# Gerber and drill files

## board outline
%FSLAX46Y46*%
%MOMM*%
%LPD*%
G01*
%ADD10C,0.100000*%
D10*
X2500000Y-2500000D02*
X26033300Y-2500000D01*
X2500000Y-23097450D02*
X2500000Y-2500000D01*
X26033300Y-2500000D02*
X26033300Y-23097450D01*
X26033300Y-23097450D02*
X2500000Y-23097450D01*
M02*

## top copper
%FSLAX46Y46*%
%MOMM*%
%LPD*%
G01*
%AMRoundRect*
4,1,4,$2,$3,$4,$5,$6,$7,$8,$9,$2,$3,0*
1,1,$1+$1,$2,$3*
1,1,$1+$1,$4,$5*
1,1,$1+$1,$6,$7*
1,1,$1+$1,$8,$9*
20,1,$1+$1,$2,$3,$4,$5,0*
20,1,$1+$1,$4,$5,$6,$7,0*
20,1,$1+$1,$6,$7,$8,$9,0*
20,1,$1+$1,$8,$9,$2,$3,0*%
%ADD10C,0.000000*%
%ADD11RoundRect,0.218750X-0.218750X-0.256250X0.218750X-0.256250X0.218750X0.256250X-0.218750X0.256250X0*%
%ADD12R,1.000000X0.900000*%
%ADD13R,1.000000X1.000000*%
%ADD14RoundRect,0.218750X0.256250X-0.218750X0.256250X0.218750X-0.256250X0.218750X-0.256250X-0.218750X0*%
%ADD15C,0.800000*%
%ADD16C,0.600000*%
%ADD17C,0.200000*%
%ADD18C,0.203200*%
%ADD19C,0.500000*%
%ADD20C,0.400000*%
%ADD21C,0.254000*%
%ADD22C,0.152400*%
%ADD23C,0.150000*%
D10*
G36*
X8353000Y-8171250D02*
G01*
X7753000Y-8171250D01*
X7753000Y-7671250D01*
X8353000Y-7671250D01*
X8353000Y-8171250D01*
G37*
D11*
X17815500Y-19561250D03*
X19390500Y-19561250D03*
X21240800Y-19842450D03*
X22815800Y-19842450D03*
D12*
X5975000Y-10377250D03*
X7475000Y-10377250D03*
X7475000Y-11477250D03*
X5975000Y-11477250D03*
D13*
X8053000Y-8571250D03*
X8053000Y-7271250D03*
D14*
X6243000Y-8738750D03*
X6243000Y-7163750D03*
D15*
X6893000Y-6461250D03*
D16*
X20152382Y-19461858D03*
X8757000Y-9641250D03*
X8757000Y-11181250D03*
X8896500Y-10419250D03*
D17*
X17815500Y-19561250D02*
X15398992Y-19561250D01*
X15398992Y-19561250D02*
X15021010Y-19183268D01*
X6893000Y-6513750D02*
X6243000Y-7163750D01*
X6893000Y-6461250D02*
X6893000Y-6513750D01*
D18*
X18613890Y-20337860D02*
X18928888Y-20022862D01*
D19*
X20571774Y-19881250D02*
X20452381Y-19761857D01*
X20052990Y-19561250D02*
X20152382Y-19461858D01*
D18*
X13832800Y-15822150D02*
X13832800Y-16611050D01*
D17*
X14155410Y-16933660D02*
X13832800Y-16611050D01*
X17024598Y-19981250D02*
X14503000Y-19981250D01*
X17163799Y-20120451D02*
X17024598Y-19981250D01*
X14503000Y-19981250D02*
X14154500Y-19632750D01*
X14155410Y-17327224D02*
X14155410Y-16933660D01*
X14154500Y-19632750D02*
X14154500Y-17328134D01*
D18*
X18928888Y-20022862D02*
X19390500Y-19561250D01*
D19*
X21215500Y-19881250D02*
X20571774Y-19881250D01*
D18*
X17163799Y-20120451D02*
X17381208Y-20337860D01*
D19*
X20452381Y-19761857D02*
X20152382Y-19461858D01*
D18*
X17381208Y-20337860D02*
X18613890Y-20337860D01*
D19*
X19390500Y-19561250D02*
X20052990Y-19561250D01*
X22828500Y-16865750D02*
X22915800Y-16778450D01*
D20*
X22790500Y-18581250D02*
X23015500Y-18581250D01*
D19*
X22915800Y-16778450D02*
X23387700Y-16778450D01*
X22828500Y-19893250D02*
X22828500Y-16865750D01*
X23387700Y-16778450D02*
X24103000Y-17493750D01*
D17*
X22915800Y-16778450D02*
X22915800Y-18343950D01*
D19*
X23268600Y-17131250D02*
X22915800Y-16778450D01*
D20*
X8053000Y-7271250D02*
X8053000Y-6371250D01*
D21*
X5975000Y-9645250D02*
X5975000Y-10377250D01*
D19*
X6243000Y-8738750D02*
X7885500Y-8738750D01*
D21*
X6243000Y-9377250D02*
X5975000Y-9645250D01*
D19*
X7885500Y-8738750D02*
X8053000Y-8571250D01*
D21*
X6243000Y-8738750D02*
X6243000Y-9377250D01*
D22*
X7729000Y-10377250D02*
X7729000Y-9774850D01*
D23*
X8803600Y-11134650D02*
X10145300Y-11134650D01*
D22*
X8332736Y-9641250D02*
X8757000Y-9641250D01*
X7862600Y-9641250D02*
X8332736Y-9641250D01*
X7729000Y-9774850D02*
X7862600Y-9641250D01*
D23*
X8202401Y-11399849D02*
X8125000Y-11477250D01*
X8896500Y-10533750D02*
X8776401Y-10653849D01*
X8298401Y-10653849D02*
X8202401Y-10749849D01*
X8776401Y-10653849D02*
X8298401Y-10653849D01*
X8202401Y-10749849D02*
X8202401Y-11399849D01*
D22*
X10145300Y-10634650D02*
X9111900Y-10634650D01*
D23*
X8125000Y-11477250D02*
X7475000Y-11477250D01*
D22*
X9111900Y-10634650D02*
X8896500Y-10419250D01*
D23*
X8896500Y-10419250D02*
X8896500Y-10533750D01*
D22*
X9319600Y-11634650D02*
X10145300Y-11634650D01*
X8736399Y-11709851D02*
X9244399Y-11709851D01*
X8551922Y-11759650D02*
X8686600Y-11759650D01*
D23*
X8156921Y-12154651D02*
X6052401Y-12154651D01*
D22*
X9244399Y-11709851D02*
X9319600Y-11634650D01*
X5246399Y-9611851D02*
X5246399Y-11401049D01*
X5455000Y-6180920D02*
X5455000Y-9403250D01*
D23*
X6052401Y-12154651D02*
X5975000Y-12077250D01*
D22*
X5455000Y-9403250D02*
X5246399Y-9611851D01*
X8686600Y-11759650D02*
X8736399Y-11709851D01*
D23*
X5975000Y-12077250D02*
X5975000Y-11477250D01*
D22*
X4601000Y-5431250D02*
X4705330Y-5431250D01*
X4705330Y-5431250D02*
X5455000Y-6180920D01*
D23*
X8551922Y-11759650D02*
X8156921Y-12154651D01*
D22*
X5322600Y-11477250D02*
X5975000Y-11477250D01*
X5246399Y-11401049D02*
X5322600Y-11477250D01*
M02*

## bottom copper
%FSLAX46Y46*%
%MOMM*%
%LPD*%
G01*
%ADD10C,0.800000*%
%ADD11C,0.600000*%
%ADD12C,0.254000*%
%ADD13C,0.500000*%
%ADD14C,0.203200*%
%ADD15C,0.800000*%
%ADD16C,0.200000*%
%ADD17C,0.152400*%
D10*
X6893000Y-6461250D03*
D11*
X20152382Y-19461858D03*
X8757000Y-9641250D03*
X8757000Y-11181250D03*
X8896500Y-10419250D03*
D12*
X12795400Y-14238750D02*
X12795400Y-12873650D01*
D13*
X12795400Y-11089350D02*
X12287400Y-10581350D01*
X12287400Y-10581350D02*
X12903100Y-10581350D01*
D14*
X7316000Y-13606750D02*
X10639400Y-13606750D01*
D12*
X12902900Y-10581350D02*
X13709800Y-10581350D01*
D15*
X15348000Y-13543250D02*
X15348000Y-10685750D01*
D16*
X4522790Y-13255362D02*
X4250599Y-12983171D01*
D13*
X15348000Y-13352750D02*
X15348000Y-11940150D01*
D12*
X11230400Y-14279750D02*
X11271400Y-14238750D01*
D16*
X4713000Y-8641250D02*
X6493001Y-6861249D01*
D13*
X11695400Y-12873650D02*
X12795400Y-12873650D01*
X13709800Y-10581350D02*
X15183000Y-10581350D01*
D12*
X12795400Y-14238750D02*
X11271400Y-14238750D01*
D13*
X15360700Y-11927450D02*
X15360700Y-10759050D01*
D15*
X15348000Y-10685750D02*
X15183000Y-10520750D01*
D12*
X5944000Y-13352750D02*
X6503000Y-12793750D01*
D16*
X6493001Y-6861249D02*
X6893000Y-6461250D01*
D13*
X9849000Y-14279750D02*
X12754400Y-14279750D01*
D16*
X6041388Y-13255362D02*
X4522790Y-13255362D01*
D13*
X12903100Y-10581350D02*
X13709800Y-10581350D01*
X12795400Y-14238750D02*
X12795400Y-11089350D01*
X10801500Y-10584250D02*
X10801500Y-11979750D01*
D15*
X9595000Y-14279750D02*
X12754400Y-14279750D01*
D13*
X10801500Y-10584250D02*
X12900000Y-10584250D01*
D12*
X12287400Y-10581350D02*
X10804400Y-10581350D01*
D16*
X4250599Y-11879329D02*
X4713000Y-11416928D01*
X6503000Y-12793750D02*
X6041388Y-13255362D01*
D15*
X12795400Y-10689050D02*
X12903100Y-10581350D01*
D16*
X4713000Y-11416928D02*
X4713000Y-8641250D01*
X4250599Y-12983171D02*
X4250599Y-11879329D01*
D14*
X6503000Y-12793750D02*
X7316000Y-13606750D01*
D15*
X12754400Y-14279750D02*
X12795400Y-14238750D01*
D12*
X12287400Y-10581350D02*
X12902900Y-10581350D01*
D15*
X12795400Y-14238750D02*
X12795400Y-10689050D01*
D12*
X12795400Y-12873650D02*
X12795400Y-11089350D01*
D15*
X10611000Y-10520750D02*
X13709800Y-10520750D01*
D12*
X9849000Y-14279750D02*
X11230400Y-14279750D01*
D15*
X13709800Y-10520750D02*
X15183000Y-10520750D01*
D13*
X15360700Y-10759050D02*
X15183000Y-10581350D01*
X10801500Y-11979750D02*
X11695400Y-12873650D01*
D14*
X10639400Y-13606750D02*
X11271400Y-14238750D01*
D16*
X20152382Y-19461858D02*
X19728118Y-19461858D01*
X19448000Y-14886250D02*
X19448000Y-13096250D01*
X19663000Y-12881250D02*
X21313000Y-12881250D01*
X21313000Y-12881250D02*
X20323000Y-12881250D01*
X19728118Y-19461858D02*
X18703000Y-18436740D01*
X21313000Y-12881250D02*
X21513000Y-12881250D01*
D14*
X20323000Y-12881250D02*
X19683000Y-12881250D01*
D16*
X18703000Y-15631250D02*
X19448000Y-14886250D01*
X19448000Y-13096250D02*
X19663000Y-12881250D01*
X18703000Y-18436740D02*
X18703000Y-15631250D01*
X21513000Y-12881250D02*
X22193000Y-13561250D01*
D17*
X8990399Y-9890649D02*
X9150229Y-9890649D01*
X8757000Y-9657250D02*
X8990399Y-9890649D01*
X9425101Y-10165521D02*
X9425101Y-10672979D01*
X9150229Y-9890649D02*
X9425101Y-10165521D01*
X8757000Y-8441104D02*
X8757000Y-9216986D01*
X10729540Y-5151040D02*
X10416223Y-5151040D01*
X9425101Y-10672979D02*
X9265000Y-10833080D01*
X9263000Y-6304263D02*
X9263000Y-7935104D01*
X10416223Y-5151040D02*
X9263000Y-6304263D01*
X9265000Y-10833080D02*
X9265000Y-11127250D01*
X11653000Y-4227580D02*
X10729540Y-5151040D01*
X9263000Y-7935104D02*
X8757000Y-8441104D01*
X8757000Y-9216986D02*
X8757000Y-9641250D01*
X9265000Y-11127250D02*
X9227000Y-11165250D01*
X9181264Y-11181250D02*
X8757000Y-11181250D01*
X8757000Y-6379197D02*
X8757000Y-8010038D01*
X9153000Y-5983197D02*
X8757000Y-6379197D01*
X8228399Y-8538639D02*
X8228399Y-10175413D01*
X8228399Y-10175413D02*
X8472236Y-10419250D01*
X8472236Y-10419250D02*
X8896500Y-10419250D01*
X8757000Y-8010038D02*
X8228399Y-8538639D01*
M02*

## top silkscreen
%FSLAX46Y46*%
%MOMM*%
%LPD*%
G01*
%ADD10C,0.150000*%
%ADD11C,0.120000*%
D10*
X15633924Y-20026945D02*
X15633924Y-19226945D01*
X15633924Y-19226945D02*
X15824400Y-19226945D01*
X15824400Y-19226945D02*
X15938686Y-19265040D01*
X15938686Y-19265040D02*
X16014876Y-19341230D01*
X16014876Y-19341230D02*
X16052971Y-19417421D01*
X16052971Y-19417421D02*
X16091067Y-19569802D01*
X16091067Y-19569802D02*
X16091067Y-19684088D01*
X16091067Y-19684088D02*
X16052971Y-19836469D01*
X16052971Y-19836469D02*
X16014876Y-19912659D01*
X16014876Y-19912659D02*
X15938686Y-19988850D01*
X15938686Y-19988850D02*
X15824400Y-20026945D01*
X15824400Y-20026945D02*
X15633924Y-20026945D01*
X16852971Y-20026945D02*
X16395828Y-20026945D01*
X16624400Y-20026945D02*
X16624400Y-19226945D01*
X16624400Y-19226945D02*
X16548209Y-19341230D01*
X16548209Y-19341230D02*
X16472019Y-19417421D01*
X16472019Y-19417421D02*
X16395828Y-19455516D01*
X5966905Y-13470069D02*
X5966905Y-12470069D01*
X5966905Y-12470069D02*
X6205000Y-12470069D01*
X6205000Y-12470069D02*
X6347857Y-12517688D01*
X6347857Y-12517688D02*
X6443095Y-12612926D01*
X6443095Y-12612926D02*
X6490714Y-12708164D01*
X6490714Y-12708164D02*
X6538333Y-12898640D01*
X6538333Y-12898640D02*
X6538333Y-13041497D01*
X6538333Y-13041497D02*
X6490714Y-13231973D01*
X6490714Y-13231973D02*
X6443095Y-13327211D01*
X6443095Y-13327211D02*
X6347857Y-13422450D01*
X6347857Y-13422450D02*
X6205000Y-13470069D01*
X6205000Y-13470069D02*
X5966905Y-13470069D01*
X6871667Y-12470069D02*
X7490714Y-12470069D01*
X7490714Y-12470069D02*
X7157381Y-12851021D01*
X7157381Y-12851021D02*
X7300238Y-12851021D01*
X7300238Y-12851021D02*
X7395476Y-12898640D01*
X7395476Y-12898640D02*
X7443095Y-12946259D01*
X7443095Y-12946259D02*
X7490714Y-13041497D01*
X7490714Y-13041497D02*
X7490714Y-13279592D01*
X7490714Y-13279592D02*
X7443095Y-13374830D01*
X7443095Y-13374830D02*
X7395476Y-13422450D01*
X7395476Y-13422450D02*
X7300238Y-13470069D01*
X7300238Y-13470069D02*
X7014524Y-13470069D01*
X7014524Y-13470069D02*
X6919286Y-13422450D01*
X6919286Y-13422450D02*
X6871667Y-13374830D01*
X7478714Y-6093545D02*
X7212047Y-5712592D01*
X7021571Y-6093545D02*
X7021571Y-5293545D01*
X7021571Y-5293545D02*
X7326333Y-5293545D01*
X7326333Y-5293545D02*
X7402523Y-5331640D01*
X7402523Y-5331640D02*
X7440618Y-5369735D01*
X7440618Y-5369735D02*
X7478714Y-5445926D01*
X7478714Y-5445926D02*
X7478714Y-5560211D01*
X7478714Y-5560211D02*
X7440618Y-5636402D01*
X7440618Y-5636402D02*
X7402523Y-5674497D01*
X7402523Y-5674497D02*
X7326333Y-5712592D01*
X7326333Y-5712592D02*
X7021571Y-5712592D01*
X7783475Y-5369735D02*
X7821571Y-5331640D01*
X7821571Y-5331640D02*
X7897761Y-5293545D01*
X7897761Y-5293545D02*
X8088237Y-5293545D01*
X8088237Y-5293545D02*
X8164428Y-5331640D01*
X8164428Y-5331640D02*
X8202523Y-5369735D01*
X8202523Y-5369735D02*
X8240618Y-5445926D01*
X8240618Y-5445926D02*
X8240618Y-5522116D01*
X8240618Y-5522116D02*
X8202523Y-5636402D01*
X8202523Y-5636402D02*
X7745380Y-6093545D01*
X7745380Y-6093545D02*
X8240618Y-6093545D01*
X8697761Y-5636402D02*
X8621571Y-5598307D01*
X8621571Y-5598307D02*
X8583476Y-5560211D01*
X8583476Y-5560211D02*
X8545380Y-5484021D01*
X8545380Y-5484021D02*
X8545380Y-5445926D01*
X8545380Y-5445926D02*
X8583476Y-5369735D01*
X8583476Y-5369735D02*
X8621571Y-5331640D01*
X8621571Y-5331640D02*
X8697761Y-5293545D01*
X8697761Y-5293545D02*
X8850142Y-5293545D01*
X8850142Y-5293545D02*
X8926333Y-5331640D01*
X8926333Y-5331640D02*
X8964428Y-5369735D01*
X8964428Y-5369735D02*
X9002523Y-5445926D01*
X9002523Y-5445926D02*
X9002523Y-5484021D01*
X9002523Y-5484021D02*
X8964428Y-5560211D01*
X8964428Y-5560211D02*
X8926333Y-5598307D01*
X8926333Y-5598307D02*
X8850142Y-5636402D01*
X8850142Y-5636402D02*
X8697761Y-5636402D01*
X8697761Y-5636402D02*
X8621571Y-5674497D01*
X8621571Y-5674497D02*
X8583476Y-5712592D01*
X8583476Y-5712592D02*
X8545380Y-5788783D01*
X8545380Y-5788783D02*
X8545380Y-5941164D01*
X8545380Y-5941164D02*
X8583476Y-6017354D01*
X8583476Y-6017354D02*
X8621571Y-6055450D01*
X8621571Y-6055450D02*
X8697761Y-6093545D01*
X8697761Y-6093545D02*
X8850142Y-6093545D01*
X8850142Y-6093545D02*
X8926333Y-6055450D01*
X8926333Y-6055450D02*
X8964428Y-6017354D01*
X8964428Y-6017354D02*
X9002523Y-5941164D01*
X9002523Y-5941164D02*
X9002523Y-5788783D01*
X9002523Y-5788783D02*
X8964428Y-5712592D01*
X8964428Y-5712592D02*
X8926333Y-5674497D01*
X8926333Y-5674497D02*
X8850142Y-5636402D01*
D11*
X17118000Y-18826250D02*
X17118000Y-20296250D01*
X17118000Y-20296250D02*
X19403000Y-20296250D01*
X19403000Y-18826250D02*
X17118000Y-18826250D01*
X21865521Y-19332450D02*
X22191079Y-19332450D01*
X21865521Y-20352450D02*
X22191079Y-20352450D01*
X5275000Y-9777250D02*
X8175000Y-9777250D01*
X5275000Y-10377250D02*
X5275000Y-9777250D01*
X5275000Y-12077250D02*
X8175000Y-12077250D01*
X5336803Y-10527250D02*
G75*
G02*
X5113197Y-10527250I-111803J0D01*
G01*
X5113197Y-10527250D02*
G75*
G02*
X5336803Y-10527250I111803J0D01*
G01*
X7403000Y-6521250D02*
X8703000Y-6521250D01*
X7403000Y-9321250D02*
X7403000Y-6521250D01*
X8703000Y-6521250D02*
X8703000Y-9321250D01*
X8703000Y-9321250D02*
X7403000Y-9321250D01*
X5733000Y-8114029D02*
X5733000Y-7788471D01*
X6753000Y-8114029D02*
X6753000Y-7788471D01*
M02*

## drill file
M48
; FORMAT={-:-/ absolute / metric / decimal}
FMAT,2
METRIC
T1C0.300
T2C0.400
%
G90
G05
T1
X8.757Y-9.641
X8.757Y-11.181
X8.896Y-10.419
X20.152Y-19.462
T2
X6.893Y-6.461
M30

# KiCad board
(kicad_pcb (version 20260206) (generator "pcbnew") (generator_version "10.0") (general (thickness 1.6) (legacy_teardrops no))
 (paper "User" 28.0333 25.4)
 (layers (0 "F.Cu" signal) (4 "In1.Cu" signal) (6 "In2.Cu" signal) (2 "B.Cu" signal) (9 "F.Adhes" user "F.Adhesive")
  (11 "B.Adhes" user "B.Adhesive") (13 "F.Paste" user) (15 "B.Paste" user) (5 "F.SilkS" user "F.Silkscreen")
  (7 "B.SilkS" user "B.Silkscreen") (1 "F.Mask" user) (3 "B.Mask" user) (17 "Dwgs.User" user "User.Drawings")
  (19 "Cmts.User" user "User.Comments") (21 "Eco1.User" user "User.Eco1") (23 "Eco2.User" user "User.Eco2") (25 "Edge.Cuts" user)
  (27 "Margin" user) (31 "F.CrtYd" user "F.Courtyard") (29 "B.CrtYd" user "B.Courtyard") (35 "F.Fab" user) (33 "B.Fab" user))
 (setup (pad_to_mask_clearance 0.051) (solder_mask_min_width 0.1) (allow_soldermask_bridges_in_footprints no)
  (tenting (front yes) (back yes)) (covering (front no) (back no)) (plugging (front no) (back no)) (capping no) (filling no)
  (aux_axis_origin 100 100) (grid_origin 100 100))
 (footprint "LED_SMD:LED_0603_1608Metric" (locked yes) (layer "F.Cu") (at 18.603 19.56125)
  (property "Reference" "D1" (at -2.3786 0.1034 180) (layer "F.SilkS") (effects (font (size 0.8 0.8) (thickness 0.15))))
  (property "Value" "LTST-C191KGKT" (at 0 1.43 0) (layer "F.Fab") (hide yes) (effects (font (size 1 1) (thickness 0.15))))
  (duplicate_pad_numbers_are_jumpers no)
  (fp_line (start -1.485 -0.735) (end -1.485 0.735) (stroke (width 0.12) (type solid)) (layer "F.SilkS"))
  (fp_line (start -1.485 0.735) (end 0.8 0.735) (stroke (width 0.12) (type solid)) (layer "F.SilkS"))
  (fp_line (start 0.8 -0.735) (end -1.485 -0.735) (stroke (width 0.12) (type solid)) (layer "F.SilkS"))
  (pad "1" smd roundrect (at -0.7875 0) (size 0.875 0.95) (layers "F.Cu" "F.Mask" "F.Paste") (roundrect_rratio 0.25) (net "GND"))
  (pad "2" smd roundrect (at 0.7875 0) (size 0.875 0.95) (layers "F.Cu" "F.Mask" "F.Paste") (roundrect_rratio 0.25) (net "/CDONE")))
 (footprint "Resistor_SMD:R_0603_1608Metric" (layer "F.Cu") (at 22.0283 19.84245)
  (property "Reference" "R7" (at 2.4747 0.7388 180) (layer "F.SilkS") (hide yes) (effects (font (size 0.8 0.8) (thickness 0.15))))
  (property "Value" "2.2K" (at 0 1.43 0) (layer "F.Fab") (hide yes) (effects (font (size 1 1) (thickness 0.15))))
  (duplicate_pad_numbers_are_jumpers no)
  (fp_line (start -0.162779 -0.51) (end 0.162779 -0.51) (stroke (width 0.12) (type solid)) (layer "F.SilkS"))
  (fp_line (start -0.162779 0.51) (end 0.162779 0.51) (stroke (width 0.12) (type solid)) (layer "F.SilkS"))
  (pad "1" smd roundrect (at -0.7875 0) (size 0.875 0.95) (layers "F.Cu" "F.Mask" "F.Paste") (roundrect_rratio 0.25) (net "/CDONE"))
  (pad "2" smd roundrect (at 0.7875 0) (size 0.875 0.95) (layers "F.Cu" "F.Mask" "F.Paste") (roundrect_rratio 0.25) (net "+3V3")))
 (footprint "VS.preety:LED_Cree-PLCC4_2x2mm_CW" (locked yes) (layer "F.Cu") (at 6.725 10.92725)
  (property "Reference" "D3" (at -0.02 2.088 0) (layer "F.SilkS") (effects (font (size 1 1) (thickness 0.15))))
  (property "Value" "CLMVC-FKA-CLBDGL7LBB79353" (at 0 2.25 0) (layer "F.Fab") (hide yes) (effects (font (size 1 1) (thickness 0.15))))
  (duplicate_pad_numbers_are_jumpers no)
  (fp_line (start -1.45 -1.15) (end 1.45 -1.15) (stroke (width 0.12) (type solid)) (layer "F.SilkS"))
  (fp_line (start -1.45 -0.55) (end -1.45 -1.15) (stroke (width 0.12) (type solid)) (layer "F.SilkS"))
  (fp_line (start -1.45 1.15) (end 1.45 1.15) (stroke (width 0.12) (type solid)) (layer "F.SilkS"))
  (fp_circle (center -1.5 -0.4) (end -1.45 -0.3) (stroke (width 0.12) (type solid)) (fill no) (layer "F.SilkS"))
  (pad "1" smd rect (at -0.75 -0.55) (size 1 0.9) (layers "F.Cu" "F.Mask" "F.Paste") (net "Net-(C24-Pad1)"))
  (pad "2" smd rect (at 0.75 -0.55) (size 1 0.9) (layers "F.Cu" "F.Mask" "F.Paste") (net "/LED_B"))
  (pad "3" smd rect (at 0.75 0.55) (size 1 0.9) (layers "F.Cu" "F.Mask" "F.Paste") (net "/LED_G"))
  (pad "4" smd rect (at -0.75 0.55) (size 1 0.9) (layers "F.Cu" "F.Mask" "F.Paste") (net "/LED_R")))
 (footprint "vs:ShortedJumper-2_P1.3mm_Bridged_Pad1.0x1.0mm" (layer "F.Cu") (at 8.053 7.92125 90)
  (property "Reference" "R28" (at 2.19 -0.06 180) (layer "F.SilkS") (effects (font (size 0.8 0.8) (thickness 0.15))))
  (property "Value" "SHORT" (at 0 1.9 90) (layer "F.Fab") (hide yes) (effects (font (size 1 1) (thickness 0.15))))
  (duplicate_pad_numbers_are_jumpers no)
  (fp_poly (pts (xy -0.25 -0.3) (xy 0.25 -0.3) (xy 0.25 0.3) (xy -0.25 0.3)) (stroke (width 0) (type solid)) (fill yes) (layer "F.Cu"))
  (fp_line (start 1.4 -0.65) (end 1.4 0.65) (stroke (width 0.12) (type solid)) (layer "F.SilkS"))
  (fp_line (start -1.4 -0.65) (end 1.4 -0.65) (stroke (width 0.12) (type solid)) (layer "F.SilkS"))
  (fp_line (start 1.4 0.65) (end -1.4 0.65) (stroke (width 0.12) (type solid)) (layer "F.SilkS"))
  (fp_line (start -1.4 0.65) (end -1.4 -0.65) (stroke (width 0.12) (type solid)) (layer "F.SilkS"))
  (pad "1" smd rect (at -0.65 0 90) (size 1 1) (layers "F.Cu" "F.Mask") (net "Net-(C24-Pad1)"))
  (pad "2" smd rect (at 0.65 0 90) (size 1 1) (layers "F.Cu" "F.Mask") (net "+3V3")))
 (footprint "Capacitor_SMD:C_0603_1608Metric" (layer "F.Cu") (at 6.243 7.95125 90)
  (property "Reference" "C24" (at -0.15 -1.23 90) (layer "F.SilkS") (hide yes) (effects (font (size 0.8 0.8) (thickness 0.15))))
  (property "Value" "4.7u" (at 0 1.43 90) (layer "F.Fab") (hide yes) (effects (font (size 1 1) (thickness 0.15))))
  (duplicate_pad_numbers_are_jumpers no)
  (fp_line (start -0.162779 -0.51) (end 0.162779 -0.51) (stroke (width 0.12) (type solid)) (layer "F.SilkS"))
  (fp_line (start -0.162779 0.51) (end 0.162779 0.51) (stroke (width 0.12) (type solid)) (layer "F.SilkS"))
  (pad "1" smd roundrect (at -0.7875 0 90) (size 0.875 0.95) (layers "F.Cu" "F.Mask" "F.Paste") (roundrect_rratio 0.25)
   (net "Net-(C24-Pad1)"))
  (pad "2" smd roundrect (at 0.7875 0 90) (size 0.875 0.95) (layers "F.Cu" "F.Mask" "F.Paste") (roundrect_rratio 0.25) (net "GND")))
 (gr_line (start 2.5 2.5) (end 26.0333 2.5) (stroke (width 0.1) (type default)) (layer "Edge.Cuts"))
 (gr_line (start 2.5 23.09745) (end 2.5 2.5) (stroke (width 0.1) (type default)) (layer "Edge.Cuts"))
 (gr_line (start 26.0333 2.5) (end 26.0333 23.09745) (stroke (width 0.1) (type default)) (layer "Edge.Cuts"))
 (gr_line (start 26.0333 23.09745) (end 2.5 23.09745) (stroke (width 0.1) (type default)) (layer "Edge.Cuts"))
 (segment (start 17.8155 19.56125) (end 15.398992 19.56125) (width 0.2) (layer "F.Cu") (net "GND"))
 (segment (start 15.398992 19.56125) (end 15.02101 19.183268) (width 0.2) (layer "F.Cu") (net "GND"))
 (segment (start 6.893 6.51375) (end 6.243 7.16375) (width 0.2) (layer "F.Cu") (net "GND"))
 (segment (start 6.893 6.46125) (end 6.893 6.51375) (width 0.2) (layer "F.Cu") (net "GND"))
 (via (at 6.893 6.46125) (size 0.8) (drill 0.4) (layers "F.Cu" "B.Cu") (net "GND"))
 (segment (start 12.7954 14.23875) (end 12.7954 12.87365) (width 0.254) (layer "B.Cu") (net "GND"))
 (segment (start 12.7954 11.08935) (end 12.2874 10.58135) (width 0.5) (layer "B.Cu") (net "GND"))
 (segment (start 12.2874 10.58135) (end 12.9031 10.58135) (width 0.5) (layer "B.Cu") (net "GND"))
 (segment (start 7.316 13.60675) (end 10.6394 13.60675) (width 0.2032) (layer "B.Cu") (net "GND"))
 (segment (start 12.9029 10.58135) (end 13.7098 10.58135) (width 0.254) (layer "B.Cu") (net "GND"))
 (segment (start 15.348 13.54325) (end 15.348 10.68575) (width 0.8) (layer "B.Cu") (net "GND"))
 (segment (start 4.52279 13.255362) (end 4.250599 12.983171) (width 0.2) (layer "B.Cu") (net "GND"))
 (segment (start 15.348 13.35275) (end 15.348 11.94015) (width 0.5) (layer "B.Cu") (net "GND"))
 (segment (start 11.2304 14.27975) (end 11.2714 14.23875) (width 0.254) (layer "B.Cu") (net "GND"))
 (segment (start 4.713 8.64125) (end 6.493001 6.861249) (width 0.2) (layer "B.Cu") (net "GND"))
 (segment (start 11.6954 12.87365) (end 12.7954 12.87365) (width 0.5) (layer "B.Cu") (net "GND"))
 (segment (start 13.7098 10.58135) (end 15.183 10.58135) (width 0.5) (layer "B.Cu") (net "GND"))
 (segment (start 12.7954 14.23875) (end 11.2714 14.23875) (width 0.254) (layer "B.Cu") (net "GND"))
 (segment (start 15.3607 11.92745) (end 15.3607 10.75905) (width 0.5) (layer "B.Cu") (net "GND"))
 (segment (start 15.348 10.68575) (end 15.183 10.52075) (width 0.8) (layer "B.Cu") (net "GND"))
 (segment (start 5.944 13.35275) (end 6.503 12.79375) (width 0.254) (layer "B.Cu") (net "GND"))
 (segment (start 6.493001 6.861249) (end 6.893 6.46125) (width 0.2) (layer "B.Cu") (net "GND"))
 (segment (start 9.849 14.27975) (end 12.7544 14.27975) (width 0.5) (layer "B.Cu") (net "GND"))
 (segment (start 6.041388 13.255362) (end 4.52279 13.255362) (width 0.2) (layer "B.Cu") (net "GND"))
 (segment (start 12.9031 10.58135) (end 13.7098 10.58135) (width 0.5) (layer "B.Cu") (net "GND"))
 (segment (start 12.7954 14.23875) (end 12.7954 11.08935) (width 0.5) (layer "B.Cu") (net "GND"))
 (segment (start 10.8015 10.58425) (end 10.8015 11.97975) (width 0.5) (layer "B.Cu") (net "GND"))
 (segment (start 9.595 14.27975) (end 12.7544 14.27975) (width 0.8) (layer "B.Cu") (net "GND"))
 (segment (start 10.8015 10.58425) (end 12.9 10.58425) (width 0.5) (layer "B.Cu") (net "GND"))
 (segment (start 12.2874 10.58135) (end 10.8044 10.58135) (width 0.254) (layer "B.Cu") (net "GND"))
 (segment (start 4.250599 11.879329) (end 4.713 11.416928) (width 0.2) (layer "B.Cu") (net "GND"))
 (segment (start 6.503 12.79375) (end 6.041388 13.255362) (width 0.2) (layer "B.Cu") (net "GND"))
 (segment (start 12.7954 10.68905) (end 12.9031 10.58135) (width 0.8) (layer "B.Cu") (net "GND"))
 (segment (start 4.713 11.416928) (end 4.713 8.64125) (width 0.2) (layer "B.Cu") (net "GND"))
 (segment (start 4.250599 12.983171) (end 4.250599 11.879329) (width 0.2) (layer "B.Cu") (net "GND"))
 (segment (start 6.503 12.79375) (end 7.316 13.60675) (width 0.2032) (layer "B.Cu") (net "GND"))
 (segment (start 12.7544 14.27975) (end 12.7954 14.23875) (width 0.8) (layer "B.Cu") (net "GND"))
 (segment (start 12.2874 10.58135) (end 12.9029 10.58135) (width 0.254) (layer "B.Cu") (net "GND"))
 (segment (start 12.7954 14.23875) (end 12.7954 10.68905) (width 0.8) (layer "B.Cu") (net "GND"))
 (segment (start 12.7954 12.87365) (end 12.7954 11.08935) (width 0.254) (layer "B.Cu") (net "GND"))
 (segment (start 10.611 10.52075) (end 13.7098 10.52075) (width 0.8) (layer "B.Cu") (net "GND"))
 (segment (start 9.849 14.27975) (end 11.2304 14.27975) (width 0.254) (layer "B.Cu") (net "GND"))
 (segment (start 13.7098 10.52075) (end 15.183 10.52075) (width 0.8) (layer "B.Cu") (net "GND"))
 (segment (start 15.3607 10.75905) (end 15.183 10.58135) (width 0.5) (layer "B.Cu") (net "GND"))
 (segment (start 10.8015 11.97975) (end 11.6954 12.87365) (width 0.5) (layer "B.Cu") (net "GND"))
 (segment (start 10.6394 13.60675) (end 11.2714 14.23875) (width 0.2032) (layer "B.Cu") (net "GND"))
 (segment (start 18.61389 20.33786) (end 18.928888 20.022862) (width 0.2032) (layer "F.Cu") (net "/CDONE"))
 (segment (start 20.571774 19.88125) (end 20.452381 19.761857) (width 0.5) (layer "F.Cu") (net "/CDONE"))
 (segment (start 20.05299 19.56125) (end 20.152382 19.461858) (width 0.5) (layer "F.Cu") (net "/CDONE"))
 (segment (start 13.8328 15.82215) (end 13.8328 16.61105) (width 0.2032) (layer "F.Cu") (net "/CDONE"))
 (segment (start 14.15541 16.93366) (end 13.8328 16.61105) (width 0.2) (layer "F.Cu") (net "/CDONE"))
 (segment (start 17.024598 19.98125) (end 14.503 19.98125) (width 0.2) (layer "F.Cu") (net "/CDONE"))
 (segment (start 17.163799 20.120451) (end 17.024598 19.98125) (width 0.2) (layer "F.Cu") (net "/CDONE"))
 (segment (start 14.503 19.98125) (end 14.1545 19.63275) (width 0.2) (layer "F.Cu") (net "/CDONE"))
 (segment (start 14.15541 17.327224) (end 14.15541 16.93366) (width 0.2) (layer "F.Cu") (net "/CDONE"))
 (segment (start 14.1545 19.63275) (end 14.1545 17.328134) (width 0.2) (layer "F.Cu") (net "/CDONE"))
 (segment (start 18.928888 20.022862) (end 19.3905 19.56125) (width 0.2032) (layer "F.Cu") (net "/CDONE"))
 (segment (start 21.2155 19.88125) (end 20.571774 19.88125) (width 0.5) (layer "F.Cu") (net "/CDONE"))
 (segment (start 17.163799 20.120451) (end 17.381208 20.33786) (width 0.2032) (layer "F.Cu") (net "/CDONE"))
 (segment (start 20.452381 19.761857) (end 20.152382 19.461858) (width 0.5) (layer "F.Cu") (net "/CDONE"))
 (segment (start 17.381208 20.33786) (end 18.61389 20.33786) (width 0.2032) (layer "F.Cu") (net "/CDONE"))
 (segment (start 19.3905 19.56125) (end 20.05299 19.56125) (width 0.5) (layer "F.Cu") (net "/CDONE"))
 (via (at 20.152382 19.461858) (size 0.6) (drill 0.3) (layers "F.Cu" "B.Cu") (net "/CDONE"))
 (segment (start 20.152382 19.461858) (end 19.728118 19.461858) (width 0.2) (layer "B.Cu") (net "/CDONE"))
 (segment (start 19.448 14.88625) (end 19.448 13.09625) (width 0.2) (layer "B.Cu") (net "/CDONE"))
 (segment (start 19.663 12.88125) (end 21.313 12.88125) (width 0.2) (layer "B.Cu") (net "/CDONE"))
 (segment (start 21.313 12.88125) (end 20.323 12.88125) (width 0.2) (layer "B.Cu") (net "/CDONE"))
 (segment (start 19.728118 19.461858) (end 18.703 18.43674) (width 0.2) (layer "B.Cu") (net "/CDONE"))
 (segment (start 21.313 12.88125) (end 21.513 12.88125) (width 0.2) (layer "B.Cu") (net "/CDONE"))
 (segment (start 20.323 12.88125) (end 19.683 12.88125) (width 0.2032) (layer "B.Cu") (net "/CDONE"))
 (segment (start 18.703 15.63125) (end 19.448 14.88625) (width 0.2) (layer "B.Cu") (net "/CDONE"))
 (segment (start 19.448 13.09625) (end 19.663 12.88125) (width 0.2) (layer "B.Cu") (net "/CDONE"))
 (segment (start 18.703 18.43674) (end 18.703 15.63125) (width 0.2) (layer "B.Cu") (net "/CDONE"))
 (segment (start 21.513 12.88125) (end 22.193 13.56125) (width 0.2) (layer "B.Cu") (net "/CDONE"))
 (segment (start 22.8285 16.86575) (end 22.9158 16.77845) (width 0.5) (layer "F.Cu") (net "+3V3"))
 (segment (start 22.7905 18.58125) (end 23.0155 18.58125) (width 0.4) (layer "F.Cu") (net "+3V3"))
 (segment (start 22.9158 16.77845) (end 23.3877 16.77845) (width 0.5) (layer "F.Cu") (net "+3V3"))
 (segment (start 22.8285 19.89325) (end 22.8285 16.86575) (width 0.5) (layer "F.Cu") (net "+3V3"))
 (segment (start 23.3877 16.77845) (end 24.103 17.49375) (width 0.5) (layer "F.Cu") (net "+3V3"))
 (segment (start 22.9158 16.77845) (end 22.9158 18.34395) (width 0.2) (layer "F.Cu") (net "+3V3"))
 (segment (start 23.2686 17.13125) (end 22.9158 16.77845) (width 0.5) (layer "F.Cu") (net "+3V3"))
 (segment (start 8.053 7.27125) (end 8.053 6.37125) (width 0.4) (layer "F.Cu") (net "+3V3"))
 (segment (start 5.975 9.64525) (end 5.975 10.37725) (width 0.254) (layer "F.Cu") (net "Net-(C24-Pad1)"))
 (segment (start 6.243 8.73875) (end 7.8855 8.73875) (width 0.5) (layer "F.Cu") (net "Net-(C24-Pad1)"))
 (segment (start 6.243 9.37725) (end 5.975 9.64525) (width 0.254) (layer "F.Cu") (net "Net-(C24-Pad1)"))
 (segment (start 7.8855 8.73875) (end 8.053 8.57125) (width 0.5) (layer "F.Cu") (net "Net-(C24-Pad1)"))
 (segment (start 6.243 8.73875) (end 6.243 9.37725) (width 0.254) (layer "F.Cu") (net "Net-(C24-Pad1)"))
 (segment (start 7.729 10.37725) (end 7.729 9.77485) (width 0.1524) (layer "F.Cu") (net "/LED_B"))
 (segment (start 8.8036 11.13465) (end 10.1453 11.13465) (width 0.15) (layer "F.Cu") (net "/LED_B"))
 (segment (start 8.332736 9.64125) (end 8.757 9.64125) (width 0.1524) (layer "F.Cu") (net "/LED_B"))
 (segment (start 7.8626 9.64125) (end 8.332736 9.64125) (width 0.1524) (layer "F.Cu") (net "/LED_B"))
 (segment (start 7.729 9.77485) (end 7.8626 9.64125) (width 0.1524) (layer "F.Cu") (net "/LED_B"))
 (via (at 8.757 9.64125) (size 0.6) (drill 0.3) (layers "F.Cu" "B.Cu") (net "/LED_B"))
 (via (at 8.757 11.18125) (size 0.6) (drill 0.3) (layers "F.Cu" "B.Cu") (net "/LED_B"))
 (segment (start 8.990399 9.890649) (end 9.150229 9.890649) (width 0.1524) (layer "B.Cu") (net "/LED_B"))
 (segment (start 8.757 9.65725) (end 8.990399 9.890649) (width 0.1524) (layer "B.Cu") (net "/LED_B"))
 (segment (start 9.425101 10.165521) (end 9.425101 10.672979) (width 0.1524) (layer "B.Cu") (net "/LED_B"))
 (segment (start 9.150229 9.890649) (end 9.425101 10.165521) (width 0.1524) (layer "B.Cu") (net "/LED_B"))
 (segment (start 8.757 8.441104) (end 8.757 9.216986) (width 0.1524) (layer "B.Cu") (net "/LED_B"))
 (segment (start 10.72954 5.15104) (end 10.416223 5.15104) (width 0.1524) (layer "B.Cu") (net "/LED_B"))
 (segment (start 9.425101 10.672979) (end 9.265 10.83308) (width 0.1524) (layer "B.Cu") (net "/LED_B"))
 (segment (start 9.263 6.304263) (end 9.263 7.935104) (width 0.1524) (layer "B.Cu") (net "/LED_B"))
 (segment (start 10.416223 5.15104) (end 9.263 6.304263) (width 0.1524) (layer "B.Cu") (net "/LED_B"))
 (segment (start 9.265 10.83308) (end 9.265 11.12725) (width 0.1524) (layer "B.Cu") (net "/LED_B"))
 (segment (start 11.653 4.22758) (end 10.72954 5.15104) (width 0.1524) (layer "B.Cu") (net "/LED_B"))
 (segment (start 9.263 7.935104) (end 8.757 8.441104) (width 0.1524) (layer "B.Cu") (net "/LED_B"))
 (segment (start 8.757 9.216986) (end 8.757 9.64125) (width 0.1524) (layer "B.Cu") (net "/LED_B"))
 (segment (start 9.265 11.12725) (end 9.227 11.16525) (width 0.1524) (layer "B.Cu") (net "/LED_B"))
 (segment (start 9.181264 11.18125) (end 8.757 11.18125) (width 0.1524) (layer "B.Cu") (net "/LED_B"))
 (segment (start 8.202401 11.399849) (end 8.125 11.47725) (width 0.15) (layer "F.Cu") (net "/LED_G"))
 (segment (start 8.8965 10.53375) (end 8.776401 10.653849) (width 0.15) (layer "F.Cu") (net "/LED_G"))
 (segment (start 8.298401 10.653849) (end 8.202401 10.749849) (width 0.15) (layer "F.Cu") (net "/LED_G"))
 (segment (start 8.776401 10.653849) (end 8.298401 10.653849) (width 0.15) (layer "F.Cu") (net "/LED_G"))
 (segment (start 8.202401 10.749849) (end 8.202401 11.399849) (width 0.15) (layer "F.Cu") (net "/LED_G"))
 (segment (start 10.1453 10.63465) (end 9.1119 10.63465) (width 0.1524) (layer "F.Cu") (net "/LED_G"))
 (segment (start 8.125 11.47725) (end 7.475 11.47725) (width 0.15) (layer "F.Cu") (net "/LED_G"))
 (segment (start 9.1119 10.63465) (end 8.8965 10.41925) (width 0.1524) (layer "F.Cu") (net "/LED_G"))
 (segment (start 8.8965 10.41925) (end 8.8965 10.53375) (width 0.15) (layer "F.Cu") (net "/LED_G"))
 (via (at 8.8965 10.41925) (size 0.6) (drill 0.3) (layers "F.Cu" "B.Cu") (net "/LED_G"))
 (segment (start 8.757 6.379197) (end 8.757 8.010038) (width 0.1524) (layer "B.Cu") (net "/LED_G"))
 (segment (start 9.153 5.983197) (end 8.757 6.379197) (width 0.1524) (layer "B.Cu") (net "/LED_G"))
 (segment (start 8.228399 8.538639) (end 8.228399 10.175413) (width 0.1524) (layer "B.Cu") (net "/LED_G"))
 (segment (start 8.228399 10.175413) (end 8.472236 10.41925) (width 0.1524) (layer "B.Cu") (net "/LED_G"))
 (segment (start 8.472236 10.41925) (end 8.8965 10.41925) (width 0.1524) (layer "B.Cu") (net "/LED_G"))
 (segment (start 8.757 8.010038) (end 8.228399 8.538639) (width 0.1524) (layer "B.Cu") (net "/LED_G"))
 (segment (start 9.3196 11.63465) (end 10.1453 11.63465) (width 0.1524) (layer "F.Cu") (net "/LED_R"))
 (segment (start 8.736399 11.709851) (end 9.244399 11.709851) (width 0.1524) (layer "F.Cu") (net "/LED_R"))
 (segment (start 8.551922 11.75965) (end 8.6866 11.75965) (width 0.1524) (layer "F.Cu") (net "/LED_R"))
 (segment (start 8.156921 12.154651) (end 6.052401 12.154651) (width 0.15) (layer "F.Cu") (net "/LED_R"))
 (segment (start 9.244399 11.709851) (end 9.3196 11.63465) (width 0.1524) (layer "F.Cu") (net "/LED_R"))
 (segment (start 5.246399 9.611851) (end 5.246399 11.401049) (width 0.1524) (layer "F.Cu") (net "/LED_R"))
 (segment (start 5.455 6.18092) (end 5.455 9.40325) (width 0.1524) (layer "F.Cu") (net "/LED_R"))
 (segment (start 6.052401 12.154651) (end 5.975 12.07725) (width 0.15) (layer "F.Cu") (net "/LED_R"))
 (segment (start 5.455 9.40325) (end 5.246399 9.611851) (width 0.1524) (layer "F.Cu") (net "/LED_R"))
 (segment (start 8.6866 11.75965) (end 8.736399 11.709851) (width 0.1524) (layer "F.Cu") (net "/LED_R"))
 (segment (start 5.975 12.07725) (end 5.975 11.47725) (width 0.15) (layer "F.Cu") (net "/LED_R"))
 (segment (start 4.601 5.43125) (end 4.70533 5.43125) (width 0.1524) (layer "F.Cu") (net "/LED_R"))
 (segment (start 4.70533 5.43125) (end 5.455 6.18092) (width 0.1524) (layer "F.Cu") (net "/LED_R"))
 (segment (start 8.551922 11.75965) (end 8.156921 12.154651) (width 0.15) (layer "F.Cu") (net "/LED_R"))
 (segment (start 5.3226 11.47725) (end 5.975 11.47725) (width 0.1524) (layer "F.Cu") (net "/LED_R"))
 (segment (start 5.246399 11.401049) (end 5.3226 11.47725) (width 0.1524) (layer "F.Cu") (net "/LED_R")))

